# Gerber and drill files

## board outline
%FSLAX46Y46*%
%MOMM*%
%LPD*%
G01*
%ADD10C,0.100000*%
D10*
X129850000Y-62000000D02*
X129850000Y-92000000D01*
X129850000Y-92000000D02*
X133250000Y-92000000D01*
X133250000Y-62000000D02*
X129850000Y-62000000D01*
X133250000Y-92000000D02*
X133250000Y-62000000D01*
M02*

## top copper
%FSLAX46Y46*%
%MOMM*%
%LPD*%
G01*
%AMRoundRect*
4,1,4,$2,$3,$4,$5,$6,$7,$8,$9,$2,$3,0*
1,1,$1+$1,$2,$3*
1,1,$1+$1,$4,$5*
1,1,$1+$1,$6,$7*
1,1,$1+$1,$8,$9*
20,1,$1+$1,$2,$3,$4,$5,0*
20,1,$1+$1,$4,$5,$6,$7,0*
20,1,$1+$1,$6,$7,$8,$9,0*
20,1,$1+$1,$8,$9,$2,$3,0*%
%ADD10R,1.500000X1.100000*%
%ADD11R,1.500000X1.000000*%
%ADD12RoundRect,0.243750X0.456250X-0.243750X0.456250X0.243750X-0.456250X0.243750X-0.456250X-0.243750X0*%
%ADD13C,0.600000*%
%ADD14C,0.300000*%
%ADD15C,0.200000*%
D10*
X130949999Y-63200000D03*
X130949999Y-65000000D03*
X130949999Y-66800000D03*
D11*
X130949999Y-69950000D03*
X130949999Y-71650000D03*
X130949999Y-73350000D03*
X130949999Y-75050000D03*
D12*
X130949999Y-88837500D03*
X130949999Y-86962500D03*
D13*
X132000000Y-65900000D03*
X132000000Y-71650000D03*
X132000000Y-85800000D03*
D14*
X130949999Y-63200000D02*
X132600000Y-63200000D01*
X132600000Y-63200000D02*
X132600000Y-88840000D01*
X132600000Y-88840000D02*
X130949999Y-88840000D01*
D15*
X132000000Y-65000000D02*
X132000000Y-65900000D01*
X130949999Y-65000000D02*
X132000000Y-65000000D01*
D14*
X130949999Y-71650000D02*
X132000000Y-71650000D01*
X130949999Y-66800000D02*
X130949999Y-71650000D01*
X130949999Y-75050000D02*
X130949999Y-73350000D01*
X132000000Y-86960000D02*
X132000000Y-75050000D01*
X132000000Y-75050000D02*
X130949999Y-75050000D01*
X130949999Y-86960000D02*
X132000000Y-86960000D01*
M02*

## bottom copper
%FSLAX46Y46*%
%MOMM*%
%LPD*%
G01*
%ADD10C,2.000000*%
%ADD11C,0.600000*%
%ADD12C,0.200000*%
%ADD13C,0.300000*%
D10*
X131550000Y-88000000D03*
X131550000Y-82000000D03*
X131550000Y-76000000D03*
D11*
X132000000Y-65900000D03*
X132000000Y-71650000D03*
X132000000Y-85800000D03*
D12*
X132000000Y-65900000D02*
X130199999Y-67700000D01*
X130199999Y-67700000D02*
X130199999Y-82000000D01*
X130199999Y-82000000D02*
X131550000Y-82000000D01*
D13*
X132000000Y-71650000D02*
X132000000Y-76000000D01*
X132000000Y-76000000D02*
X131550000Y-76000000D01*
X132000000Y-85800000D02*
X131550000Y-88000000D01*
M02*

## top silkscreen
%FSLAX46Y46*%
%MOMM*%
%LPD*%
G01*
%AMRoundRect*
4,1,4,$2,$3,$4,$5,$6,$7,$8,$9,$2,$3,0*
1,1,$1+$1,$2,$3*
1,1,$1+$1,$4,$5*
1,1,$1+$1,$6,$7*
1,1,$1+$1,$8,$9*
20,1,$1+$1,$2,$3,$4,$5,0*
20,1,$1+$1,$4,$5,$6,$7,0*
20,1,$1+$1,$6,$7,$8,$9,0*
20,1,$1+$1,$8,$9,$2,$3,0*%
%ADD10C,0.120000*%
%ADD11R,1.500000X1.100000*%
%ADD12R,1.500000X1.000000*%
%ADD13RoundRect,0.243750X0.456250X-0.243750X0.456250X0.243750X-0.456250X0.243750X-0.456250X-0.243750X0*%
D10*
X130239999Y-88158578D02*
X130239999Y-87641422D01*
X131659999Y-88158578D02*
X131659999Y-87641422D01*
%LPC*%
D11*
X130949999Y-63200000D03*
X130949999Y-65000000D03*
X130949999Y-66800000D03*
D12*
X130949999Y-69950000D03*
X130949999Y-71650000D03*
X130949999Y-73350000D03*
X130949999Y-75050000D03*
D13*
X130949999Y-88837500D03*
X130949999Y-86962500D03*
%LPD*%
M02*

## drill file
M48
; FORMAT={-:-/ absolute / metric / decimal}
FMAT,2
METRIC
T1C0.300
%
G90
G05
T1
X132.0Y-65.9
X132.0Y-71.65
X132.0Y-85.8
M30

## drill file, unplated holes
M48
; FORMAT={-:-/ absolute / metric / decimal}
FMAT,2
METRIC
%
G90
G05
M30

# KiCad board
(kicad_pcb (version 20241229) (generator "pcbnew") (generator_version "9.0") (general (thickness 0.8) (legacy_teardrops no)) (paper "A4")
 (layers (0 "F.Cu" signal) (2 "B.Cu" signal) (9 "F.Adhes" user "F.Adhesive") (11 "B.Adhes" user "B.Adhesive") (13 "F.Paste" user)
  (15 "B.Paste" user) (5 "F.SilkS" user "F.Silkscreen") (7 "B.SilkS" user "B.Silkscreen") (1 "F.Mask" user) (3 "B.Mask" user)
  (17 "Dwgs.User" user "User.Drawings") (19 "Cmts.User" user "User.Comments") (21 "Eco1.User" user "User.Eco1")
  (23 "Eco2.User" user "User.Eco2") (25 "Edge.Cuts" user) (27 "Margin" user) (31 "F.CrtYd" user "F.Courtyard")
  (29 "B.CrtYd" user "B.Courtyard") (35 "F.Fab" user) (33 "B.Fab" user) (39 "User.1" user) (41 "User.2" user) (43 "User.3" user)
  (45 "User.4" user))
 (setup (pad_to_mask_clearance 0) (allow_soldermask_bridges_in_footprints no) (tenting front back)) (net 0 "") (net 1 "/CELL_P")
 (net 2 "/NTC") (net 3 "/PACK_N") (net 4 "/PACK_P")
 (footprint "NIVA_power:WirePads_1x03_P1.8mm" (layer "F.Cu") (at 130.949999 65)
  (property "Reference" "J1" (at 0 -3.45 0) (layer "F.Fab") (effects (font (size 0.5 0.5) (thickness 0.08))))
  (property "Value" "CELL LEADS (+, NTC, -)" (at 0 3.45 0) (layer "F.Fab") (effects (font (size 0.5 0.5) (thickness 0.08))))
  (pad "1" smd rect (at 0 -1.8) (size 1.5 1.1) (layers "F.Cu" "F.Mask") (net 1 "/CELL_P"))
  (pad "2" smd rect (at 0 0) (size 1.5 1.1) (layers "F.Cu" "F.Mask") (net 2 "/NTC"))
  (pad "3" smd rect (at 0 1.8) (size 1.5 1.1) (layers "F.Cu" "F.Mask") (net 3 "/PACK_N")))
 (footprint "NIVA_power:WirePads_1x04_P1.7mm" (layer "F.Cu") (at 130.949999 72.5)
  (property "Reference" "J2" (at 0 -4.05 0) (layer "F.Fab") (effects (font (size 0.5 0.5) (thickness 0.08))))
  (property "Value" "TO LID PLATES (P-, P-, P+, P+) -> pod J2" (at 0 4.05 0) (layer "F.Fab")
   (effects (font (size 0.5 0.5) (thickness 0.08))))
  (pad "1" smd rect (at 0 -2.55) (size 1.5 1) (layers "F.Cu" "F.Mask") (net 3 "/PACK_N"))
  (pad "2" smd rect (at 0 -0.85) (size 1.5 1) (layers "F.Cu" "F.Mask") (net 3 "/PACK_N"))
  (pad "3" smd rect (at 0 0.85) (size 1.5 1) (layers "F.Cu" "F.Mask") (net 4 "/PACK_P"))
  (pad "4" smd rect (at 0 2.55) (size 1.5 1) (layers "F.Cu" "F.Mask") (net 4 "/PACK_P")))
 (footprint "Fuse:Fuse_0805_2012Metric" (layer "F.Cu") (at 130.949999 87.9 90)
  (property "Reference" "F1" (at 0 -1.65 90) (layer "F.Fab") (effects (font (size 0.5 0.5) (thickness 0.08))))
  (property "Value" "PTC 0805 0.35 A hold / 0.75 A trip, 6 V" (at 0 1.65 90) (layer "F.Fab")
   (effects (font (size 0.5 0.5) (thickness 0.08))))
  (fp_line (start -0.258578 -0.71) (end 0.258578 -0.71) (stroke (width 0.12) (type solid)) (layer "F.SilkS"))
  (fp_line (start -0.258578 0.71) (end 0.258578 0.71) (stroke (width 0.12) (type solid)) (layer "F.SilkS"))
  (pad "1" smd roundrect (at -0.9375 0 90) (size 0.975 1.4) (layers "F.Cu" "F.Mask" "F.Paste") (roundrect_rratio 0.25) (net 1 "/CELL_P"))
  (pad "2" smd roundrect (at 0.9375 0 90) (size 0.975 1.4) (layers "F.Cu" "F.Mask" "F.Paste") (roundrect_rratio 0.25) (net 4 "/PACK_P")))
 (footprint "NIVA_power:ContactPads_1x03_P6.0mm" (layer "B.Cu") (at 131.55 82)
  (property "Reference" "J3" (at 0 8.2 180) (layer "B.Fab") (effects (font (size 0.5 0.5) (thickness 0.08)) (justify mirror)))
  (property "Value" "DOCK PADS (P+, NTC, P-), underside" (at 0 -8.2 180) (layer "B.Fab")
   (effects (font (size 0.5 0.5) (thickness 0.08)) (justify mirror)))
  (pad "1" smd circle (at 0 6) (size 2 2) (layers "B.Cu" "B.Mask") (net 4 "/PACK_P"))
  (pad "2" smd circle (at 0 0) (size 2 2) (layers "B.Cu" "B.Mask") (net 2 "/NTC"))
  (pad "3" smd circle (at 0 -6) (size 2 2) (layers "B.Cu" "B.Mask") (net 3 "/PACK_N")))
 (gr_line (start 129.85 62) (end 129.85 92) (stroke (width 0.1) (type default)) (layer "Edge.Cuts"))
 (gr_line (start 129.85 92) (end 133.25 92) (stroke (width 0.1) (type default)) (layer "Edge.Cuts"))
 (gr_line (start 133.25 62) (end 129.85 62) (stroke (width 0.1) (type default)) (layer "Edge.Cuts"))
 (gr_line (start 133.25 92) (end 133.25 62) (stroke (width 0.1) (type default)) (layer "Edge.Cuts"))
 (segment (start 130.949999 63.2) (end 132.6 63.2) (width 0.3) (layer "F.Cu") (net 1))
 (segment (start 132.6 63.2) (end 132.6 88.84) (width 0.3) (layer "F.Cu") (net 1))
 (segment (start 132.6 88.84) (end 130.949999 88.84) (width 0.3) (layer "F.Cu") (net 1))
 (segment (start 132 65) (end 132 65.9) (width 0.2) (layer "F.Cu") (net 2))
 (segment (start 130.949999 65) (end 132 65) (width 0.2) (layer "F.Cu") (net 2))
 (via (at 132 65.9) (size 0.6) (drill 0.3) (layers "F.Cu" "B.Cu") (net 2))
 (segment (start 132 65.9) (end 130.199999 67.7) (width 0.2) (layer "B.Cu") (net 2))
 (segment (start 130.199999 67.7) (end 130.199999 82) (width 0.2) (layer "B.Cu") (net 2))
 (segment (start 130.199999 82) (end 131.55 82) (width 0.2) (layer "B.Cu") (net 2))
 (segment (start 130.949999 71.65) (end 132 71.65) (width 0.3) (layer "F.Cu") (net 3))
 (segment (start 130.949999 66.8) (end 130.949999 71.65) (width 0.3) (layer "F.Cu") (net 3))
 (via (at 132 71.65) (size 0.6) (drill 0.3) (layers "F.Cu" "B.Cu") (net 3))
 (segment (start 132 71.65) (end 132 76) (width 0.3) (layer "B.Cu") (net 3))
 (segment (start 132 76) (end 131.55 76) (width 0.3) (layer "B.Cu") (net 3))
 (segment (start 130.949999 75.05) (end 130.949999 73.35) (width 0.3) (layer "F.Cu") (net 4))
 (segment (start 132 86.96) (end 132 75.05) (width 0.3) (layer "F.Cu") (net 4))
 (segment (start 132 75.05) (end 130.949999 75.05) (width 0.3) (layer "F.Cu") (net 4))
 (segment (start 130.949999 86.96) (end 132 86.96) (width 0.3) (layer "F.Cu") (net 4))
 (via (at 132 85.8) (size 0.6) (drill 0.3) (layers "F.Cu" "B.Cu") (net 4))
 (segment (start 132 85.8) (end 131.55 88) (width 0.3) (layer "B.Cu") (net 4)))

